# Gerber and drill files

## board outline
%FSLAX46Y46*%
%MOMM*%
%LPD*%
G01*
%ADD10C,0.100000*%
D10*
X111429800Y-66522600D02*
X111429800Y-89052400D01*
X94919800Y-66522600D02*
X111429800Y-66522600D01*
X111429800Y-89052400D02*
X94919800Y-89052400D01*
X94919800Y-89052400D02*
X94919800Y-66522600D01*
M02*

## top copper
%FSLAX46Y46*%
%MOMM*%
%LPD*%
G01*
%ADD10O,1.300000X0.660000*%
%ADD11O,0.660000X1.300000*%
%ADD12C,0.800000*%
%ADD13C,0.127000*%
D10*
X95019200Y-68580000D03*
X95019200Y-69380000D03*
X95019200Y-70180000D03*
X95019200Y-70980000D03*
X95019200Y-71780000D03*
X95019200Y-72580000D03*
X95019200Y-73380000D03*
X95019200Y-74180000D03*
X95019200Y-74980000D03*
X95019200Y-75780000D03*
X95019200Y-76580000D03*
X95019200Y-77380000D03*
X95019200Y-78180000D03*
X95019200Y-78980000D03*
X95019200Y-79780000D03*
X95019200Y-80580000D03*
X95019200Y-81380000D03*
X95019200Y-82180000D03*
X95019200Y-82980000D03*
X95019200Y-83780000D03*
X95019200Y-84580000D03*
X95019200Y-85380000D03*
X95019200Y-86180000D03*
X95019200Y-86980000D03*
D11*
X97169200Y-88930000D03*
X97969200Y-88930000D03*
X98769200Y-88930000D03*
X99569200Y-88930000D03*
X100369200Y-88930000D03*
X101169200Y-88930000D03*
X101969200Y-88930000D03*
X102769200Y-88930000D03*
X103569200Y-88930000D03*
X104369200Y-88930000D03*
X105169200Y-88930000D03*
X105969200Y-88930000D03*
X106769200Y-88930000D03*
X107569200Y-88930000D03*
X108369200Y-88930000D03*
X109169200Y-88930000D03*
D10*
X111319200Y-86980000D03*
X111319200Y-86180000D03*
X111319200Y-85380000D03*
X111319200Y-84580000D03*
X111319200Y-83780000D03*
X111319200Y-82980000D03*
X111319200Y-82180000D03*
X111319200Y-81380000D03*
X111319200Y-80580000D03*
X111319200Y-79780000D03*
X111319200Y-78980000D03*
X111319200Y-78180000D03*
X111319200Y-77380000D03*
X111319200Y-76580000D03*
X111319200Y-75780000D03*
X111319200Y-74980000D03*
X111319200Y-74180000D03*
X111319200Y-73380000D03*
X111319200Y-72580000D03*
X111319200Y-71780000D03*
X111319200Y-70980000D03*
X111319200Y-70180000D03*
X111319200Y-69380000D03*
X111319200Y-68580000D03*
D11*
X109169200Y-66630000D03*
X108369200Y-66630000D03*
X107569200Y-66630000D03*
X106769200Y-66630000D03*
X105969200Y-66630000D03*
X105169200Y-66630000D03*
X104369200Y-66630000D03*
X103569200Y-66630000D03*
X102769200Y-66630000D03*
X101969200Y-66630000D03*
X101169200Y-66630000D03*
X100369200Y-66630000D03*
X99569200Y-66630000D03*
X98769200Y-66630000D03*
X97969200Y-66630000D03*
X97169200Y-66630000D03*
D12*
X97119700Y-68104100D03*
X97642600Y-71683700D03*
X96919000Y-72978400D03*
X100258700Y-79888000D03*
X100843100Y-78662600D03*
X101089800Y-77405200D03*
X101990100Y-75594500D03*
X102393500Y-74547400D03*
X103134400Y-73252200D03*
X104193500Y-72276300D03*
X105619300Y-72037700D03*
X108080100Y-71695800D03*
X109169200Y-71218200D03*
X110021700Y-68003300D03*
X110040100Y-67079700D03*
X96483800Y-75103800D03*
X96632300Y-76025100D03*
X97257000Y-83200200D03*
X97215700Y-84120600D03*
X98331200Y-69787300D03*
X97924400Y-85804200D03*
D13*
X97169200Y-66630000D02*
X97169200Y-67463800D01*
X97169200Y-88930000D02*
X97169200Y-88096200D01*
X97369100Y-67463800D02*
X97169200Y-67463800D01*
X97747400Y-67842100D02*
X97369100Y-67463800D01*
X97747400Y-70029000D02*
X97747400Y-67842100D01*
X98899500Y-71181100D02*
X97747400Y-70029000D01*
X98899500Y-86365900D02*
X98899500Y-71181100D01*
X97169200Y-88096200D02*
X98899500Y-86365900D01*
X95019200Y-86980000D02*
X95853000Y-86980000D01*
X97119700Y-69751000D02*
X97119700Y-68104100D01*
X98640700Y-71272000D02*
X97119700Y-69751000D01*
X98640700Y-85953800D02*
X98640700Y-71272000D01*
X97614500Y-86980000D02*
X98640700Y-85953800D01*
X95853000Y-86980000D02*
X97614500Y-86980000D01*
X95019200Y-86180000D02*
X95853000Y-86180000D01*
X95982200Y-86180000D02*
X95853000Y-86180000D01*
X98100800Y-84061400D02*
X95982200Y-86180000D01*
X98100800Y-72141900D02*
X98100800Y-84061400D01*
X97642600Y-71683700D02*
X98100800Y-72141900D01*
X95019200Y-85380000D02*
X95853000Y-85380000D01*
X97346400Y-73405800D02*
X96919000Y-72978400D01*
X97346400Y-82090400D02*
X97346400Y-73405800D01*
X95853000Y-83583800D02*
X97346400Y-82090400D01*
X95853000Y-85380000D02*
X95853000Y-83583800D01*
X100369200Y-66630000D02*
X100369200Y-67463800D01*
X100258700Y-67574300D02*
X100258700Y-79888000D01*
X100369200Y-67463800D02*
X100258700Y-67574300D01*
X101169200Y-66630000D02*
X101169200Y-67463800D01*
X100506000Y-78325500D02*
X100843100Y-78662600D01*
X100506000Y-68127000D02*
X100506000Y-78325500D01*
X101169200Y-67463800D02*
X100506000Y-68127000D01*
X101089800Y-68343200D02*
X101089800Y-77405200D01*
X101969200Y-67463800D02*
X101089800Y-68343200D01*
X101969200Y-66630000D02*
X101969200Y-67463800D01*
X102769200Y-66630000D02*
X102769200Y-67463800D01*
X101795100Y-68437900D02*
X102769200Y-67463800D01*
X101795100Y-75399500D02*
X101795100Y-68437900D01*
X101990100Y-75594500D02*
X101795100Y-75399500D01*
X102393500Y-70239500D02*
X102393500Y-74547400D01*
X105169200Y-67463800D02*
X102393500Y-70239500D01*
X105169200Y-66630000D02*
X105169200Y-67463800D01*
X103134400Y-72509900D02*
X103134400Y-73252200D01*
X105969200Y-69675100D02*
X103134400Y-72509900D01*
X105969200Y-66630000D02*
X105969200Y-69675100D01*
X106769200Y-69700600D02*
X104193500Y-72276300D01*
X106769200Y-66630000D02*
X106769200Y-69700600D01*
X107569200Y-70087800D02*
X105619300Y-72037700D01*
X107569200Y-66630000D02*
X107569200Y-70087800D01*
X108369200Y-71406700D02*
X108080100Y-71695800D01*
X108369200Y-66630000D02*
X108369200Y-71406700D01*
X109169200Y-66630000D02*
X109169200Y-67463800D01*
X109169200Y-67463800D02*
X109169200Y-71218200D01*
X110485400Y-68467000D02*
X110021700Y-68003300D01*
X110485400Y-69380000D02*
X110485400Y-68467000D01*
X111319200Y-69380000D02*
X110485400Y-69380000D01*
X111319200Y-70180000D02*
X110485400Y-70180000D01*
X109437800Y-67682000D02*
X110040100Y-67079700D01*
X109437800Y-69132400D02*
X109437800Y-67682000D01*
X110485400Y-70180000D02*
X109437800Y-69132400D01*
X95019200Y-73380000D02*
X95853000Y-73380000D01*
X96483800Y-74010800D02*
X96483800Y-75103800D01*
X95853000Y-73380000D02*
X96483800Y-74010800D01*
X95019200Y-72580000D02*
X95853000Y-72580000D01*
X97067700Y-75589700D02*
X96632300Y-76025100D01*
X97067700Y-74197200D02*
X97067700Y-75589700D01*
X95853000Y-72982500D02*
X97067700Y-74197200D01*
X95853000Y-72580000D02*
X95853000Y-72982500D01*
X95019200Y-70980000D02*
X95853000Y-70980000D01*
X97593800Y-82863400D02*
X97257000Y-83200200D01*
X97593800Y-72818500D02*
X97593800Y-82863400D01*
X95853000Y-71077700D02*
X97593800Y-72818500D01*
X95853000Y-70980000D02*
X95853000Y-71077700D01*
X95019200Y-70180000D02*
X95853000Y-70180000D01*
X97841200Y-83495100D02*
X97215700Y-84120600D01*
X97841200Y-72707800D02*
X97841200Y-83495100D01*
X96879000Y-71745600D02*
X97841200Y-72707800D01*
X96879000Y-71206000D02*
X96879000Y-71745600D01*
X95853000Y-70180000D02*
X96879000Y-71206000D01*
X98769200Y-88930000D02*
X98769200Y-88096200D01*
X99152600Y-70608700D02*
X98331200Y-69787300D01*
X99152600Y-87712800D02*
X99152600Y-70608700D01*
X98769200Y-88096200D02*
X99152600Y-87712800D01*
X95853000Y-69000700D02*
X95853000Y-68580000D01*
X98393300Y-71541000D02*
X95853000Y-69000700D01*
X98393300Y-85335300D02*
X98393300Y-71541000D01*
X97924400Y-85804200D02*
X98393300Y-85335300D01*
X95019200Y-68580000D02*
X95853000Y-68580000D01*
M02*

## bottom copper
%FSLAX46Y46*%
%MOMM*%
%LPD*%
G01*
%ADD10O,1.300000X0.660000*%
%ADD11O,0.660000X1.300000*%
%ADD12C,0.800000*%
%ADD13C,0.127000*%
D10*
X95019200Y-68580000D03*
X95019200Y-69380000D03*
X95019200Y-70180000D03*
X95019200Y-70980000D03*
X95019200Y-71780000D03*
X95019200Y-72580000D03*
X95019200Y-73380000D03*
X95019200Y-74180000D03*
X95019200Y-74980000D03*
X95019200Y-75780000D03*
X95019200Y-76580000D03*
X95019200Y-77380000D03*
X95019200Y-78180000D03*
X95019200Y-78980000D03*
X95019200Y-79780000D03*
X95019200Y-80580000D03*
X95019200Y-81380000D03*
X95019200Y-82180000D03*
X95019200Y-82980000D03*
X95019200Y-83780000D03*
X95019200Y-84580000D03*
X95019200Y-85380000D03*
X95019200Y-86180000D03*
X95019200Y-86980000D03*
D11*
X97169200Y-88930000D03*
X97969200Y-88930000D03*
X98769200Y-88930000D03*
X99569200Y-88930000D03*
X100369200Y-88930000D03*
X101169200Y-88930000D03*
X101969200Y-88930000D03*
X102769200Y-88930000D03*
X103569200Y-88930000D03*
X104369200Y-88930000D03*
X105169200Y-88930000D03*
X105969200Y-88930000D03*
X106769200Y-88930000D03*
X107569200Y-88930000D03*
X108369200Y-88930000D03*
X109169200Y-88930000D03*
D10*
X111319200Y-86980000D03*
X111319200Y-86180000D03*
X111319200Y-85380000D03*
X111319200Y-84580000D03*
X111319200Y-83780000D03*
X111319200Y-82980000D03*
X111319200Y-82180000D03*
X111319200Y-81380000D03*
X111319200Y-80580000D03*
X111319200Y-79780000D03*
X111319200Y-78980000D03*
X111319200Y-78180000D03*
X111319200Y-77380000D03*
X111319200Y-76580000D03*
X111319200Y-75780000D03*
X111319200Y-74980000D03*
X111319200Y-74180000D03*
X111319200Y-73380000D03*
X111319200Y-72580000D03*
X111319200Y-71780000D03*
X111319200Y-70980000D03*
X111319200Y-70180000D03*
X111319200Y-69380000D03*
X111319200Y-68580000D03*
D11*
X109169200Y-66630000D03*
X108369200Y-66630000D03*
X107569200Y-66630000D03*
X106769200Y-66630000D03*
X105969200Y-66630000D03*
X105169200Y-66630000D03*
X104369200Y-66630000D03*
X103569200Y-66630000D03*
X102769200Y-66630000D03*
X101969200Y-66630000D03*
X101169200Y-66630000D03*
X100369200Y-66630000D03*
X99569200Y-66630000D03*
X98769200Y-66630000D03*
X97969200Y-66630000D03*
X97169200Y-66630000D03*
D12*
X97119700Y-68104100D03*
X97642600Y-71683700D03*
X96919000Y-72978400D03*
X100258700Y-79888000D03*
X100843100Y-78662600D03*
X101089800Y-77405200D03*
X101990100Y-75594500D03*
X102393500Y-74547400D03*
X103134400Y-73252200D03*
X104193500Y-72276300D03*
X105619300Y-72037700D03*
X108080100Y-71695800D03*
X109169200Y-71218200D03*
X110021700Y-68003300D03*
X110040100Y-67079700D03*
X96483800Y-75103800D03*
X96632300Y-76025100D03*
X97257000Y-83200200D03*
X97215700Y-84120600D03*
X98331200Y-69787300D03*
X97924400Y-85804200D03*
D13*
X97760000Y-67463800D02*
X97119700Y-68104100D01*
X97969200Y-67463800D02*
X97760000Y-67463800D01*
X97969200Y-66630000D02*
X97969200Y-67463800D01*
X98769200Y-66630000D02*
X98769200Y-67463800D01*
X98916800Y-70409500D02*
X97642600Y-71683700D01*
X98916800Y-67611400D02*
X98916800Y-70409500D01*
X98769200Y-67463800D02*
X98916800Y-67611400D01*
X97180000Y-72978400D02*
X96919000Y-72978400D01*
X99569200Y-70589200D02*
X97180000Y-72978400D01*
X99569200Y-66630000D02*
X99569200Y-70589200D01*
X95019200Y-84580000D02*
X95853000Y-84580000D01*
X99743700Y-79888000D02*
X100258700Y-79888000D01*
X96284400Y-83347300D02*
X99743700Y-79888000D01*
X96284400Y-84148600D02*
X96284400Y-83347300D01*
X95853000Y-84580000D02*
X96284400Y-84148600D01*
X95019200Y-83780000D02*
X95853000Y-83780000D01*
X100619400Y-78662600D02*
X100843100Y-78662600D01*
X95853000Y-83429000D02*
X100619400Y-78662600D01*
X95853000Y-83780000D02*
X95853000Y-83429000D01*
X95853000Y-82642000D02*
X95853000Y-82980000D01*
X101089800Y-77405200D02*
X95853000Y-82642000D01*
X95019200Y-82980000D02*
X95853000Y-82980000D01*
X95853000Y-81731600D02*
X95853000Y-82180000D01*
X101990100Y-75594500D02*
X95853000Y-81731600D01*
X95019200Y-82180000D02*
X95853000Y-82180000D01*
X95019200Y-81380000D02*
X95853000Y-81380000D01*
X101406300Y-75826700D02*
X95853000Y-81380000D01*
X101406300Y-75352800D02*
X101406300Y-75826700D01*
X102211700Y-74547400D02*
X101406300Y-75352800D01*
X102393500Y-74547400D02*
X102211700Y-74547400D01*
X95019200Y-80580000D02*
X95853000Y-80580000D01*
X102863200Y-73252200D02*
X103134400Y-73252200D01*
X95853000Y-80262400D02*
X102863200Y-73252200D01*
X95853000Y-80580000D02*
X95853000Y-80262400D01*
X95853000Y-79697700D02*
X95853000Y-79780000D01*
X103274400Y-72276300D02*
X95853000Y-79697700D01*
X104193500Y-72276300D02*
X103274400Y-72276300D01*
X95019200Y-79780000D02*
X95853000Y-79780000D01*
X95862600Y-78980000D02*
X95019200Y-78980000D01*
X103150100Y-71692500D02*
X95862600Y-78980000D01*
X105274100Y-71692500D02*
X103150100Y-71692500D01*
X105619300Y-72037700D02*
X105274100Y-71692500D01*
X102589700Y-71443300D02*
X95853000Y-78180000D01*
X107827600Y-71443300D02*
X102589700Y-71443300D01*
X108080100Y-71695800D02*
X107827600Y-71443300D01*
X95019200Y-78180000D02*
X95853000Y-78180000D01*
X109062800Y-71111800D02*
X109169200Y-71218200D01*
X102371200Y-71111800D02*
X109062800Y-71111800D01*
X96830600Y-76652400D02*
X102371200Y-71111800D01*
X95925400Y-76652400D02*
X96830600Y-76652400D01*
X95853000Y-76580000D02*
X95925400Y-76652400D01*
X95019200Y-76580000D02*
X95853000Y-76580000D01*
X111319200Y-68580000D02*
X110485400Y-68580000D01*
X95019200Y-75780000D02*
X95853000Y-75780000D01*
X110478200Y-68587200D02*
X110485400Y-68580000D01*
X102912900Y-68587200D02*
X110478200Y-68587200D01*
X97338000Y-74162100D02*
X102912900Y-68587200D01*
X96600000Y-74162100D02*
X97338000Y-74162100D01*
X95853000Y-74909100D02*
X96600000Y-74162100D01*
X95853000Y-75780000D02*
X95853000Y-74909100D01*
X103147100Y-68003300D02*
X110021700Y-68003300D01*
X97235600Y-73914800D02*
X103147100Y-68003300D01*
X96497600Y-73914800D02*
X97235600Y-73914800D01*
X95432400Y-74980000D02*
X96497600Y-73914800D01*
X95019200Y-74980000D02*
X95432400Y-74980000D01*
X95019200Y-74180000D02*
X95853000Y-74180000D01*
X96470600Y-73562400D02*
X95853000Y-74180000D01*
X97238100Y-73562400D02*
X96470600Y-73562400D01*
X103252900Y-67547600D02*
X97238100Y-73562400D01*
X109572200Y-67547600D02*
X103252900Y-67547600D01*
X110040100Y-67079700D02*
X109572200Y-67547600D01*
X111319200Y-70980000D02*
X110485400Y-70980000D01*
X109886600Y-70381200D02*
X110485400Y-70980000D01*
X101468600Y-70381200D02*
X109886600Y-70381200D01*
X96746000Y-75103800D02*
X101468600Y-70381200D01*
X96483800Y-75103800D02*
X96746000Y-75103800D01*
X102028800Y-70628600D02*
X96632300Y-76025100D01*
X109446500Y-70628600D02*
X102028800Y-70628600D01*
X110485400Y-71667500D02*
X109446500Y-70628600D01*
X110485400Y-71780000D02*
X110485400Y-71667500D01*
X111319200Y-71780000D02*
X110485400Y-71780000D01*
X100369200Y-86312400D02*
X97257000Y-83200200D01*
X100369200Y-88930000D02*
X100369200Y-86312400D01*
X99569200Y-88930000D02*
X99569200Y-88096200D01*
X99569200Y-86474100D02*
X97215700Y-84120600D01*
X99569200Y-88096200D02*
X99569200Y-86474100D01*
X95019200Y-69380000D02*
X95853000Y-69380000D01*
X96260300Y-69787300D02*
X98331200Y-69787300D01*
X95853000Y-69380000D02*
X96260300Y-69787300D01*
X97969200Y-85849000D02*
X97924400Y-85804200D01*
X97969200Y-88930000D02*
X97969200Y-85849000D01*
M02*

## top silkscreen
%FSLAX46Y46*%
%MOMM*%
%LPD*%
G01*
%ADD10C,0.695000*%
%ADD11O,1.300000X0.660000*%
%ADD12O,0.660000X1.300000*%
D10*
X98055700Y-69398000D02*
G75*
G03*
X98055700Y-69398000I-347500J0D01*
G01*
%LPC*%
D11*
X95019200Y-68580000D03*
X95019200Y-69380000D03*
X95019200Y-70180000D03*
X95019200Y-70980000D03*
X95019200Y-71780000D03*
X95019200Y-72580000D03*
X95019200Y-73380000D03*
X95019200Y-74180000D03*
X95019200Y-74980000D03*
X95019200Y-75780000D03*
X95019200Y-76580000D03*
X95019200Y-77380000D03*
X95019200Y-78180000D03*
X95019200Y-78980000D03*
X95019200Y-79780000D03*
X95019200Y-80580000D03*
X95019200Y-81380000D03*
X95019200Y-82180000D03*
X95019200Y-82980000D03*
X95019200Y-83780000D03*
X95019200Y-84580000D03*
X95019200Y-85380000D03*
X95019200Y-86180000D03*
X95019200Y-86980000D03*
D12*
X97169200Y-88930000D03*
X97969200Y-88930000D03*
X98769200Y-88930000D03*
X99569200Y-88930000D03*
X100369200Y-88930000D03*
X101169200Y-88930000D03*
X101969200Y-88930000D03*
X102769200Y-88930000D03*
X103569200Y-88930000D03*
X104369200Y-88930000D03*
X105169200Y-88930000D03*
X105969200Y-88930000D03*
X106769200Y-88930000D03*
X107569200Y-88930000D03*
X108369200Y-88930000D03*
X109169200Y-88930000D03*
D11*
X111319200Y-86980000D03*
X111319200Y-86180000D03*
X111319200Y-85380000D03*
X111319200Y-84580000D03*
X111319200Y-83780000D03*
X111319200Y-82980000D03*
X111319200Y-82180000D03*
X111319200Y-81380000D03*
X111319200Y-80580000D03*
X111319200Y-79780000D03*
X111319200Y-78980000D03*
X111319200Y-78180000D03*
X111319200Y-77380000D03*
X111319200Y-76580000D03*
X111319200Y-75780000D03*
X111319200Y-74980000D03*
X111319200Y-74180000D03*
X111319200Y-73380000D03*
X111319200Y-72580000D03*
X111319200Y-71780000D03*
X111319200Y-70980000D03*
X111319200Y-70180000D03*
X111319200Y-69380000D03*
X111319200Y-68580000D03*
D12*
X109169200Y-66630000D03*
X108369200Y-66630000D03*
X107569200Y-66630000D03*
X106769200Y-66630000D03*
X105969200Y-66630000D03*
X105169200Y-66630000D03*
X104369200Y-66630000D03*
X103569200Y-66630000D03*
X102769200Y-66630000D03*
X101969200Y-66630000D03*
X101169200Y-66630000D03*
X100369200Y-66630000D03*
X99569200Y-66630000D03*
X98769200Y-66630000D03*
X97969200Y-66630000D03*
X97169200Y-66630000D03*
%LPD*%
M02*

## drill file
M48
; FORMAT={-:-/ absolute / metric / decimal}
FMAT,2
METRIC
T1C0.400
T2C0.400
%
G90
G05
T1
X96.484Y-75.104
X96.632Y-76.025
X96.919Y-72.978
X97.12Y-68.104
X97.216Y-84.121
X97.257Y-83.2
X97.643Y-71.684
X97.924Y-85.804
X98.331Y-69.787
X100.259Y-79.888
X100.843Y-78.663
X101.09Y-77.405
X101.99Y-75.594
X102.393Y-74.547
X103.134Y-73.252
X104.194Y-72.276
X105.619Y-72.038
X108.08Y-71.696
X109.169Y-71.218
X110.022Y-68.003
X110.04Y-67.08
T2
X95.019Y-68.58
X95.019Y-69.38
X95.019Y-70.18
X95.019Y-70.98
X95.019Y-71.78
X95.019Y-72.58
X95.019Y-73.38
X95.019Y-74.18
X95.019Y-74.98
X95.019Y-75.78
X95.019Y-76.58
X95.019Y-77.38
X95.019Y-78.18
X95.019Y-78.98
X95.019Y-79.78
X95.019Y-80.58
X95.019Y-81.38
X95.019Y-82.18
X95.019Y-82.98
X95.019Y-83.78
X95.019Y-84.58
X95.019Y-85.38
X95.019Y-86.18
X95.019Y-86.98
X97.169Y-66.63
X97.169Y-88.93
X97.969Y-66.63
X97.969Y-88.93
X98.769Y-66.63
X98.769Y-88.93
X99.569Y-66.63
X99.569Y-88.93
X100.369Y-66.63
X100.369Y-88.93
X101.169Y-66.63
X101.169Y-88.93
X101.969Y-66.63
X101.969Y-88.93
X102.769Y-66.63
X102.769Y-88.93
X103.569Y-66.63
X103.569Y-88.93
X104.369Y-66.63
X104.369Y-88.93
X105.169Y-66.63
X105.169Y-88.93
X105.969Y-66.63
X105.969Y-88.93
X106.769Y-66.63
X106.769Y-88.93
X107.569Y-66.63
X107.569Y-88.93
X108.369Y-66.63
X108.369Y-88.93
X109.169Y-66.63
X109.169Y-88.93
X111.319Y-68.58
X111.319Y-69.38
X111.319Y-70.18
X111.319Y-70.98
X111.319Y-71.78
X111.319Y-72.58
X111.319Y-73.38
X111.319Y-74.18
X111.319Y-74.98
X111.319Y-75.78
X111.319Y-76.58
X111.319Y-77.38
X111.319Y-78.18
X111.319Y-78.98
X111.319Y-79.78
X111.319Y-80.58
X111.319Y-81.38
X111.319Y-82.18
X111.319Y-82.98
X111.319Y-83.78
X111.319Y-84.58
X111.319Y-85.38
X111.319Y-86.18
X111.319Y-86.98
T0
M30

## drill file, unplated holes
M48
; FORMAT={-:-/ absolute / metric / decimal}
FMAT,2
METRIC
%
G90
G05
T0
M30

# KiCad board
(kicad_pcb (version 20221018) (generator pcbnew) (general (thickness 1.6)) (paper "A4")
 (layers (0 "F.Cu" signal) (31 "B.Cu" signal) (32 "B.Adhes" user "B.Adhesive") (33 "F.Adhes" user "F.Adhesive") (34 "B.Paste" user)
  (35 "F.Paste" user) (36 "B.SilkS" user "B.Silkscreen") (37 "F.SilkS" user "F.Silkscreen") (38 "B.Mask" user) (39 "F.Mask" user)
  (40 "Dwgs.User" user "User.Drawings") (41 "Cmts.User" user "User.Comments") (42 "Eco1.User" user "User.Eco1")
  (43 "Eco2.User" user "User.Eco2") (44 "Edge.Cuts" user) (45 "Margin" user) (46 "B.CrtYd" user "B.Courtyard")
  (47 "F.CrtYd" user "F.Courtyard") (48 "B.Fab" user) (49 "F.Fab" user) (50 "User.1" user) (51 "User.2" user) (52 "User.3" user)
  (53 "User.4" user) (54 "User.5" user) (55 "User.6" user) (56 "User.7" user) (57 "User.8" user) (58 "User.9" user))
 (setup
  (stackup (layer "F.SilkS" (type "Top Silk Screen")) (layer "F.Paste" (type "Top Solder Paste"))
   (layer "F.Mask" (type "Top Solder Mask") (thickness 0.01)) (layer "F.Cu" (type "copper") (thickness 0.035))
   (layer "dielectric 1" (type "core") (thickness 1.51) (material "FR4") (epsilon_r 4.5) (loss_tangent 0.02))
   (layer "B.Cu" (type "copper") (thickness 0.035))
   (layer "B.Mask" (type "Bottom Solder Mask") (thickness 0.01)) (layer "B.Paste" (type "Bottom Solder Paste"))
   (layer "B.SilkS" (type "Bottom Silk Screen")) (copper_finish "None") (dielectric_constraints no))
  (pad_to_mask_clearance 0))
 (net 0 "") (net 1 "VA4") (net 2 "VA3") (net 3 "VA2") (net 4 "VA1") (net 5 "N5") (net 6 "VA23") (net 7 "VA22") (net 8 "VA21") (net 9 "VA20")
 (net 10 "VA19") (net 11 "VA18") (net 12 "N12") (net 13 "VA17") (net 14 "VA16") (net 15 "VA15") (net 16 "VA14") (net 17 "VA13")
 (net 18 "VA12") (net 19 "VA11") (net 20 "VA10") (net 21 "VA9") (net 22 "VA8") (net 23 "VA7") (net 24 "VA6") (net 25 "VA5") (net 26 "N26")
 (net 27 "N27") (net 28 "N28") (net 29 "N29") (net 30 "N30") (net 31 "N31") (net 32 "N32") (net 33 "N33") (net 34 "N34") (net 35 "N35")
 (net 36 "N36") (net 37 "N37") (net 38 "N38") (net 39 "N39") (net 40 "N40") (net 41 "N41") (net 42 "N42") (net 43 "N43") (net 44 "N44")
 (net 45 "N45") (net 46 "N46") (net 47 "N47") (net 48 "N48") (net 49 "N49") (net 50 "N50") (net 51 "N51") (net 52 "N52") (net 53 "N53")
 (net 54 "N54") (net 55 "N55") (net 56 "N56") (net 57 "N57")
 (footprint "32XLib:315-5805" (layer "F.Cu") (at 103.1692 77.78)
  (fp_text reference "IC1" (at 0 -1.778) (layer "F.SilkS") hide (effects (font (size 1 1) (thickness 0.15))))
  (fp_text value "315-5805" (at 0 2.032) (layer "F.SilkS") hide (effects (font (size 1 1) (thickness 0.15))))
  (fp_circle (center -5.461 -8.382) (end -4.826 -8.382) (stroke (width 0.12) (type solid)) (fill solid) (layer "F.SilkS"))
  (pad "1" thru_hole oval (at -8.15 -9.2) (size 1.3 0.66) (drill 0.4) (layers "*.Cu" "*.Mask") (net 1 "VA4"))
  (pad "2" thru_hole oval (at -8.15 -8.4) (size 1.3 0.66) (drill 0.4) (layers "*.Cu" "*.Mask") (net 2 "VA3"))
  (pad "3" thru_hole oval (at -8.15 -7.6) (size 1.3 0.66) (drill 0.4) (layers "*.Cu" "*.Mask") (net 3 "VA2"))
  (pad "4" thru_hole oval (at -8.15 -6.8) (size 1.3 0.66) (drill 0.4) (layers "*.Cu" "*.Mask") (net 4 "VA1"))
  (pad "5" thru_hole oval (at -8.15 -6) (size 1.3 0.66) (drill 0.4) (layers "*.Cu" "*.Mask") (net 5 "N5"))
  (pad "6" thru_hole oval (at -8.15 -5.2) (size 1.3 0.66) (drill 0.4) (layers "*.Cu" "*.Mask") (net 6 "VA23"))
  (pad "7" thru_hole oval (at -8.15 -4.4) (size 1.3 0.66) (drill 0.4) (layers "*.Cu" "*.Mask") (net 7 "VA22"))
  (pad "8" thru_hole oval (at -8.15 -3.6) (size 1.3 0.66) (drill 0.4) (layers "*.Cu" "*.Mask") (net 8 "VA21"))
  (pad "9" thru_hole oval (at -8.15 -2.8) (size 1.3 0.66) (drill 0.4) (layers "*.Cu" "*.Mask") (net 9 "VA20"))
  (pad "10" thru_hole oval (at -8.15 -2) (size 1.3 0.66) (drill 0.4) (layers "*.Cu" "*.Mask") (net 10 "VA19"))
  (pad "11" thru_hole oval (at -8.15 -1.2) (size 1.3 0.66) (drill 0.4) (layers "*.Cu" "*.Mask") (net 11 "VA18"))
  (pad "12" thru_hole oval (at -8.15 -0.4) (size 1.3 0.66) (drill 0.4) (layers "*.Cu" "*.Mask") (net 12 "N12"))
  (pad "13" thru_hole oval (at -8.15 0.4) (size 1.3 0.66) (drill 0.4) (layers "*.Cu" "*.Mask") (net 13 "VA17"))
  (pad "14" thru_hole oval (at -8.15 1.2) (size 1.3 0.66) (drill 0.4) (layers "*.Cu" "*.Mask") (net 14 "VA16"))
  (pad "15" thru_hole oval (at -8.15 2) (size 1.3 0.66) (drill 0.4) (layers "*.Cu" "*.Mask") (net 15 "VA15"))
  (pad "16" thru_hole oval (at -8.15 2.8) (size 1.3 0.66) (drill 0.4) (layers "*.Cu" "*.Mask") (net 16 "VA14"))
  (pad "17" thru_hole oval (at -8.15 3.6) (size 1.3 0.66) (drill 0.4) (layers "*.Cu" "*.Mask") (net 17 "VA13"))
  (pad "18" thru_hole oval (at -8.15 4.4) (size 1.3 0.66) (drill 0.4) (layers "*.Cu" "*.Mask") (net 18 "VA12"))
  (pad "19" thru_hole oval (at -8.15 5.2) (size 1.3 0.66) (drill 0.4) (layers "*.Cu" "*.Mask") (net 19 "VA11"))
  (pad "20" thru_hole oval (at -8.15 6) (size 1.3 0.66) (drill 0.4) (layers "*.Cu" "*.Mask") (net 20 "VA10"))
  (pad "21" thru_hole oval (at -8.15 6.8) (size 1.3 0.66) (drill 0.4) (layers "*.Cu" "*.Mask") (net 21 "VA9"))
  (pad "22" thru_hole oval (at -8.15 7.6) (size 1.3 0.66) (drill 0.4) (layers "*.Cu" "*.Mask") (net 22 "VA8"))
  (pad "23" thru_hole oval (at -8.15 8.4) (size 1.3 0.66) (drill 0.4) (layers "*.Cu" "*.Mask") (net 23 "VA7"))
  (pad "24" thru_hole oval (at -8.15 9.2) (size 1.3 0.66) (drill 0.4) (layers "*.Cu" "*.Mask") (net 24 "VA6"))
  (pad "25" thru_hole oval (at -6 11.15 90) (size 1.3 0.66) (drill 0.4) (layers "*.Cu" "*.Mask") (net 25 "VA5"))
  (pad "26" thru_hole oval (at -5.2 11.15 90) (size 1.3 0.66) (drill 0.4) (layers "*.Cu" "*.Mask") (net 1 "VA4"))
  (pad "27" thru_hole oval (at -4.4 11.15 90) (size 1.3 0.66) (drill 0.4) (layers "*.Cu" "*.Mask") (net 2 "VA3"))
  (pad "28" thru_hole oval (at -3.6 11.15 90) (size 1.3 0.66) (drill 0.4) (layers "*.Cu" "*.Mask") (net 3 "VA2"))
  (pad "29" thru_hole oval (at -2.8 11.15 90) (size 1.3 0.66) (drill 0.4) (layers "*.Cu" "*.Mask") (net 4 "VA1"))
  (pad "30" thru_hole oval (at -2 11.15 90) (size 1.3 0.66) (drill 0.4) (layers "*.Cu" "*.Mask") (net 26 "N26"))
  (pad "31" thru_hole oval (at -1.2 11.15 90) (size 1.3 0.66) (drill 0.4) (layers "*.Cu" "*.Mask") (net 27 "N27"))
  (pad "32" thru_hole oval (at -0.4 11.15 90) (size 1.3 0.66) (drill 0.4) (layers "*.Cu" "*.Mask") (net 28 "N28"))
  (pad "33" thru_hole oval (at 0.4 11.15 90) (size 1.3 0.66) (drill 0.4) (layers "*.Cu" "*.Mask") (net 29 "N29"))
  (pad "34" thru_hole oval (at 1.2 11.15 90) (size 1.3 0.66) (drill 0.4) (layers "*.Cu" "*.Mask") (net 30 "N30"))
  (pad "35" thru_hole oval (at 2 11.15 90) (size 1.3 0.66) (drill 0.4) (layers "*.Cu" "*.Mask") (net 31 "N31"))
  (pad "36" thru_hole oval (at 2.8 11.15 90) (size 1.3 0.66) (drill 0.4) (layers "*.Cu" "*.Mask") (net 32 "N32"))
  (pad "37" thru_hole oval (at 3.6 11.15 90) (size 1.3 0.66) (drill 0.4) (layers "*.Cu" "*.Mask") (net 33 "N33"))
  (pad "38" thru_hole oval (at 4.4 11.15 90) (size 1.3 0.66) (drill 0.4) (layers "*.Cu" "*.Mask") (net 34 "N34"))
  (pad "39" thru_hole oval (at 5.2 11.15 90) (size 1.3 0.66) (drill 0.4) (layers "*.Cu" "*.Mask") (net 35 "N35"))
  (pad "40" thru_hole oval (at 6 11.15 90) (size 1.3 0.66) (drill 0.4) (layers "*.Cu" "*.Mask") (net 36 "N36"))
  (pad "41" thru_hole oval (at 8.15 9.2) (size 1.3 0.66) (drill 0.4) (layers "*.Cu" "*.Mask") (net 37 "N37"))
  (pad "42" thru_hole oval (at 8.15 8.4) (size 1.3 0.66) (drill 0.4) (layers "*.Cu" "*.Mask") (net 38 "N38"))
  (pad "43" thru_hole oval (at 8.15 7.6) (size 1.3 0.66) (drill 0.4) (layers "*.Cu" "*.Mask") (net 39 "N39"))
  (pad "44" thru_hole oval (at 8.15 6.8) (size 1.3 0.66) (drill 0.4) (layers "*.Cu" "*.Mask") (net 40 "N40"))
  (pad "45" thru_hole oval (at 8.15 6) (size 1.3 0.66) (drill 0.4) (layers "*.Cu" "*.Mask") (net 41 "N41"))
  (pad "46" thru_hole oval (at 8.15 5.2) (size 1.3 0.66) (drill 0.4) (layers "*.Cu" "*.Mask") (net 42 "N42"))
  (pad "47" thru_hole oval (at 8.15 4.4) (size 1.3 0.66) (drill 0.4) (layers "*.Cu" "*.Mask") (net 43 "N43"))
  (pad "48" thru_hole oval (at 8.15 3.6) (size 1.3 0.66) (drill 0.4) (layers "*.Cu" "*.Mask") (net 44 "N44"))
  (pad "49" thru_hole oval (at 8.15 2.8) (size 1.3 0.66) (drill 0.4) (layers "*.Cu" "*.Mask") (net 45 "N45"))
  (pad "50" thru_hole oval (at 8.15 2) (size 1.3 0.66) (drill 0.4) (layers "*.Cu" "*.Mask") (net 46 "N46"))
  (pad "51" thru_hole oval (at 8.15 1.2) (size 1.3 0.66) (drill 0.4) (layers "*.Cu" "*.Mask") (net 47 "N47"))
  (pad "52" thru_hole oval (at 8.15 0.4) (size 1.3 0.66) (drill 0.4) (layers "*.Cu" "*.Mask") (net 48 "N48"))
  (pad "53" thru_hole oval (at 8.15 -0.4) (size 1.3 0.66) (drill 0.4) (layers "*.Cu" "*.Mask") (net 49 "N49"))
  (pad "54" thru_hole oval (at 8.15 -1.2) (size 1.3 0.66) (drill 0.4) (layers "*.Cu" "*.Mask") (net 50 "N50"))
  (pad "55" thru_hole oval (at 8.15 -2) (size 1.3 0.66) (drill 0.4) (layers "*.Cu" "*.Mask") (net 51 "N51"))
  (pad "56" thru_hole oval (at 8.15 -2.8) (size 1.3 0.66) (drill 0.4) (layers "*.Cu" "*.Mask") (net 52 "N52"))
  (pad "57" thru_hole oval (at 8.15 -3.6) (size 1.3 0.66) (drill 0.4) (layers "*.Cu" "*.Mask") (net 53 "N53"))
  (pad "58" thru_hole oval (at 8.15 -4.4) (size 1.3 0.66) (drill 0.4) (layers "*.Cu" "*.Mask") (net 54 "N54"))
  (pad "59" thru_hole oval (at 8.15 -5.2) (size 1.3 0.66) (drill 0.4) (layers "*.Cu" "*.Mask") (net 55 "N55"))
  (pad "60" thru_hole oval (at 8.15 -6) (size 1.3 0.66) (drill 0.4) (layers "*.Cu" "*.Mask") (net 6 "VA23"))
  (pad "61" thru_hole oval (at 8.15 -6.8) (size 1.3 0.66) (drill 0.4) (layers "*.Cu" "*.Mask") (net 7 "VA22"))
  (pad "62" thru_hole oval (at 8.15 -7.6) (size 1.3 0.66) (drill 0.4) (layers "*.Cu" "*.Mask") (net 8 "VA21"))
  (pad "63" thru_hole oval (at 8.15 -8.4) (size 1.3 0.66) (drill 0.4) (layers "*.Cu" "*.Mask") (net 9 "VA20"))
  (pad "64" thru_hole oval (at 8.15 -9.2) (size 1.3 0.66) (drill 0.4) (layers "*.Cu" "*.Mask") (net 10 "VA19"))
  (pad "65" thru_hole oval (at 6 -11.15 90) (size 1.3 0.66) (drill 0.4) (layers "*.Cu" "*.Mask") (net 11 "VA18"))
  (pad "66" thru_hole oval (at 5.2 -11.15 90) (size 1.3 0.66) (drill 0.4) (layers "*.Cu" "*.Mask") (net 13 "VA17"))
  (pad "67" thru_hole oval (at 4.4 -11.15 90) (size 1.3 0.66) (drill 0.4) (layers "*.Cu" "*.Mask") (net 14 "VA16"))
  (pad "68" thru_hole oval (at 3.6 -11.15 90) (size 1.3 0.66) (drill 0.4) (layers "*.Cu" "*.Mask") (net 15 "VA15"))
  (pad "69" thru_hole oval (at 2.8 -11.15 90) (size 1.3 0.66) (drill 0.4) (layers "*.Cu" "*.Mask") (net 16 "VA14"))
  (pad "70" thru_hole oval (at 2 -11.15 90) (size 1.3 0.66) (drill 0.4) (layers "*.Cu" "*.Mask") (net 17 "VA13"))
  (pad "71" thru_hole oval (at 1.2 -11.15 90) (size 1.3 0.66) (drill 0.4) (layers "*.Cu" "*.Mask") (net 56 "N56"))
  (pad "72" thru_hole oval (at 0.4 -11.15 90) (size 1.3 0.66) (drill 0.4) (layers "*.Cu" "*.Mask") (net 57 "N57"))
  (pad "73" thru_hole oval (at -0.4 -11.15 90) (size 1.3 0.66) (drill 0.4) (layers "*.Cu" "*.Mask") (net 18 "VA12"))
  (pad "74" thru_hole oval (at -1.2 -11.15 90) (size 1.3 0.66) (drill 0.4) (layers "*.Cu" "*.Mask") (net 19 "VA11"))
  (pad "75" thru_hole oval (at -2 -11.15 90) (size 1.3 0.66) (drill 0.4) (layers "*.Cu" "*.Mask") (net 20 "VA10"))
  (pad "76" thru_hole oval (at -2.8 -11.15 90) (size 1.3 0.66) (drill 0.4) (layers "*.Cu" "*.Mask") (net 21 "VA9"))
  (pad "77" thru_hole oval (at -3.6 -11.15 90) (size 1.3 0.66) (drill 0.4) (layers "*.Cu" "*.Mask") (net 22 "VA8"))
  (pad "78" thru_hole oval (at -4.4 -11.15 90) (size 1.3 0.66) (drill 0.4) (layers "*.Cu" "*.Mask") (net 23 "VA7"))
  (pad "79" thru_hole oval (at -5.2 -11.15 90) (size 1.3 0.66) (drill 0.4) (layers "*.Cu" "*.Mask") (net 24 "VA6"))
  (pad "80" thru_hole oval (at -6 -11.15 90) (size 1.3 0.66) (drill 0.4) (layers "*.Cu" "*.Mask") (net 25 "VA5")))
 (gr_line (start 94.9198 89.0524) (end 94.9198 66.5226) (stroke (width 0.1) (type default)) (layer "Edge.Cuts"))
 (gr_line (start 111.4298 66.5226) (end 111.4298 89.0524) (stroke (width 0.1) (type default)) (layer "Edge.Cuts"))
 (gr_line (start 94.9198 66.5226) (end 111.4298 66.5226) (stroke (width 0.1) (type default)) (layer "Edge.Cuts"))
 (gr_line (start 111.4298 89.0524) (end 94.9198 89.0524) (stroke (width 0.1) (type default)) (layer "Edge.Cuts"))
 (segment (start 98.3933 71.541) (end 95.853 69.0007) (width 0.127) (layer "F.Cu") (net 1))
 (segment (start 98.3933 85.3353) (end 98.3933 71.541) (width 0.127) (layer "F.Cu") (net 1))
 (segment (start 95.853 69.0007) (end 95.853 68.58) (width 0.127) (layer "F.Cu") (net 1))
 (segment (start 95.0192 68.58) (end 95.853 68.58) (width 0.127) (layer "F.Cu") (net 1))
 (segment (start 97.9244 85.8042) (end 98.3933 85.3353) (width 0.127) (layer "F.Cu") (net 1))
 (via (at 97.9244 85.8042) (size 0.8) (drill 0.4) (layers "F.Cu" "B.Cu") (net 1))
 (segment (start 97.9692 85.849) (end 97.9244 85.8042) (width 0.127) (layer "B.Cu") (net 1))
 (segment (start 97.9692 88.93) (end 97.9692 85.849) (width 0.127) (layer "B.Cu") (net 1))
 (segment (start 98.7692 88.93) (end 98.7692 88.0962) (width 0.127) (layer "F.Cu") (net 2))
 (segment (start 98.7692 88.0962) (end 99.1526 87.7128) (width 0.127) (layer "F.Cu") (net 2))
 (segment (start 99.1526 70.6087) (end 98.3312 69.7873) (width 0.127) (layer "F.Cu") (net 2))
 (segment (start 99.1526 87.7128) (end 99.1526 70.6087) (width 0.127) (layer "F.Cu") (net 2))
 (via (at 98.3312 69.7873) (size 0.8) (drill 0.4) (layers "F.Cu" "B.Cu") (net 2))
 (segment (start 95.853 69.38) (end 96.2603 69.7873) (width 0.127) (layer "B.Cu") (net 2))
 (segment (start 95.0192 69.38) (end 95.853 69.38) (width 0.127) (layer "B.Cu") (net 2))
 (segment (start 96.2603 69.7873) (end 98.3312 69.7873) (width 0.127) (layer "B.Cu") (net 2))
 (segment (start 95.853 70.18) (end 96.879 71.206) (width 0.127) (layer "F.Cu") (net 3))
 (segment (start 97.8412 72.7078) (end 97.8412 83.4951) (width 0.127) (layer "F.Cu") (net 3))
 (segment (start 96.879 71.206) (end 96.879 71.7456) (width 0.127) (layer "F.Cu") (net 3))
 (segment (start 95.0192 70.18) (end 95.853 70.18) (width 0.127) (layer "F.Cu") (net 3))
 (segment (start 96.879 71.7456) (end 97.8412 72.7078) (width 0.127) (layer "F.Cu") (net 3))
 (segment (start 97.8412 83.4951) (end 97.2157 84.1206) (width 0.127) (layer "F.Cu") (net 3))
 (via (at 97.2157 84.1206) (size 0.8) (drill 0.4) (layers "F.Cu" "B.Cu") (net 3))
 (segment (start 99.5692 88.0962) (end 99.5692 86.4741) (width 0.127) (layer "B.Cu") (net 3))
 (segment (start 99.5692 86.4741) (end 97.2157 84.1206) (width 0.127) (layer "B.Cu") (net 3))
 (segment (start 99.5692 88.93) (end 99.5692 88.0962) (width 0.127) (layer "B.Cu") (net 3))
 (segment (start 97.5938 82.8634) (end 97.257 83.2002) (width 0.127) (layer "F.Cu") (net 4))
 (segment (start 97.5938 72.8185) (end 97.5938 82.8634) (width 0.127) (layer "F.Cu") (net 4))
 (segment (start 95.853 71.0777) (end 97.5938 72.8185) (width 0.127) (layer "F.Cu") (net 4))
 (segment (start 95.0192 70.98) (end 95.853 70.98) (width 0.127) (layer "F.Cu") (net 4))
 (segment (start 95.853 70.98) (end 95.853 71.0777) (width 0.127) (layer "F.Cu") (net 4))
 (via (at 97.257 83.2002) (size 0.8) (drill 0.4) (layers "F.Cu" "B.Cu") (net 4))
 (segment (start 100.3692 86.3124) (end 97.257 83.2002) (width 0.127) (layer "B.Cu") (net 4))
 (segment (start 100.3692 88.93) (end 100.3692 86.3124) (width 0.127) (layer "B.Cu") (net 4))
 (segment (start 95.853 72.58) (end 95.853 72.9825) (width 0.127) (layer "F.Cu") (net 6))
 (segment (start 95.853 72.9825) (end 97.0677 74.1972) (width 0.127) (layer "F.Cu") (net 6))
 (segment (start 95.0192 72.58) (end 95.853 72.58) (width 0.127) (layer "F.Cu") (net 6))
 (segment (start 97.0677 74.1972) (end 97.0677 75.5897) (width 0.127) (layer "F.Cu") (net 6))
 (segment (start 97.0677 75.5897) (end 96.6323 76.0251) (width 0.127) (layer "F.Cu") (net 6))
 (via (at 96.6323 76.0251) (size 0.8) (drill 0.4) (layers "F.Cu" "B.Cu") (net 6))
 (segment (start 111.3192 71.78) (end 110.4854 71.78) (width 0.127) (layer "B.Cu") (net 6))
 (segment (start 110.4854 71.78) (end 110.4854 71.6675) (width 0.127) (layer "B.Cu") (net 6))
 (segment (start 109.4465 70.6286) (end 102.0288 70.6286) (width 0.127) (layer "B.Cu") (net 6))
 (segment (start 102.0288 70.6286) (end 96.6323 76.0251) (width 0.127) (layer "B.Cu") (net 6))
 (segment (start 110.4854 71.6675) (end 109.4465 70.6286) (width 0.127) (layer "B.Cu") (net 6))
 (segment (start 95.0192 73.38) (end 95.853 73.38) (width 0.127) (layer "F.Cu") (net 7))
 (segment (start 96.4838 74.0108) (end 96.4838 75.1038) (width 0.127) (layer "F.Cu") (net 7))
 (segment (start 95.853 73.38) (end 96.4838 74.0108) (width 0.127) (layer "F.Cu") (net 7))
 (via (at 96.4838 75.1038) (size 0.8) (drill 0.4) (layers "F.Cu" "B.Cu") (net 7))
 (segment (start 96.746 75.1038) (end 101.4686 70.3812) (width 0.127) (layer "B.Cu") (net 7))
 (segment (start 96.4838 75.1038) (end 96.746 75.1038) (width 0.127) (layer "B.Cu") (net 7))
 (segment (start 111.3192 70.98) (end 110.4854 70.98) (width 0.127) (layer "B.Cu") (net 7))
 (segment (start 101.4686 70.3812) (end 109.8866 70.3812) (width 0.127) (layer "B.Cu") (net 7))
 (segment (start 109.8866 70.3812) (end 110.4854 70.98) (width 0.127) (layer "B.Cu") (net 7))
 (segment (start 109.4378 69.1324) (end 109.4378 67.682) (width 0.127) (layer "F.Cu") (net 8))
 (segment (start 109.4378 67.682) (end 110.0401 67.0797) (width 0.127) (layer "F.Cu") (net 8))
 (segment (start 110.4854 70.18) (end 109.4378 69.1324) (width 0.127) (layer "F.Cu") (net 8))
 (segment (start 111.3192 70.18) (end 110.4854 70.18) (width 0.127) (layer "F.Cu") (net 8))
 (via (at 110.0401 67.0797) (size 0.8) (drill 0.4) (layers "F.Cu" "B.Cu") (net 8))
 (segment (start 96.4706 73.5624) (end 95.853 74.18) (width 0.127) (layer "B.Cu") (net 8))
 (segment (start 95.0192 74.18) (end 95.853 74.18) (width 0.127) (layer "B.Cu") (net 8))
 (segment (start 103.2529 67.5476) (end 97.2381 73.5624) (width 0.127) (layer "B.Cu") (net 8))
 (segment (start 109.5722 67.5476) (end 103.2529 67.5476) (width 0.127) (layer "B.Cu") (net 8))
 (segment (start 110.0401 67.0797) (end 109.5722 67.5476) (width 0.127) (layer "B.Cu") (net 8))
 (segment (start 97.2381 73.5624) (end 96.4706 73.5624) (width 0.127) (layer "B.Cu") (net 8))
 (segment (start 110.4854 68.467) (end 110.0217 68.0033) (width 0.127) (layer "F.Cu") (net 9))
 (segment (start 110.4854 69.38) (end 110.4854 68.467) (width 0.127) (layer "F.Cu") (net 9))
 (segment (start 111.3192 69.38) (end 110.4854 69.38) (width 0.127) (layer "F.Cu") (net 9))
 (via (at 110.0217 68.0033) (size 0.8) (drill 0.4) (layers "F.Cu" "B.Cu") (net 9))
 (segment (start 103.1471 68.0033) (end 110.0217 68.0033) (width 0.127) (layer "B.Cu") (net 9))
 (segment (start 97.2356 73.9148) (end 103.1471 68.0033) (width 0.127) (layer "B.Cu") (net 9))
 (segment (start 96.4976 73.9148) (end 97.2356 73.9148) (width 0.127) (layer "B.Cu") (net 9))
 (segment (start 95.4324 74.98) (end 96.4976 73.9148) (width 0.127) (layer "B.Cu") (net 9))
 (segment (start 95.0192 74.98) (end 95.4324 74.98) (width 0.127) (layer "B.Cu") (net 9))
 (segment (start 97.338 74.1621) (end 102.9129 68.5872) (width 0.127) (layer "B.Cu") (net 10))
 (segment (start 110.4782 68.5872) (end 110.4854 68.58) (width 0.127) (layer "B.Cu") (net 10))
 (segment (start 102.9129 68.5872) (end 110.4782 68.5872) (width 0.127) (layer "B.Cu") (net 10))
 (segment (start 95.853 75.78) (end 95.853 74.9091) (width 0.127) (layer "B.Cu") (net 10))
 (segment (start 111.3192 68.58) (end 110.4854 68.58) (width 0.127) (layer "B.Cu") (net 10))
 (segment (start 95.853 74.9091) (end 96.6 74.1621) (width 0.127) (layer "B.Cu") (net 10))
 (segment (start 96.6 74.1621) (end 97.338 74.1621) (width 0.127) (layer "B.Cu") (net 10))
 (segment (start 95.0192 75.78) (end 95.853 75.78) (width 0.127) (layer "B.Cu") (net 10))
 (segment (start 109.1692 67.4638) (end 109.1692 71.2182) (width 0.127) (layer "F.Cu") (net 11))
 (segment (start 109.1692 66.63) (end 109.1692 67.4638) (width 0.127) (layer "F.Cu") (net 11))
 (via (at 109.1692 71.2182) (size 0.8) (drill 0.4) (layers "F.Cu" "B.Cu") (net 11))
 (segment (start 95.0192 76.58) (end 95.853 76.58) (width 0.127) (layer "B.Cu") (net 11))
 (segment (start 95.853 76.58) (end 95.9254 76.6524) (width 0.127) (layer "B.Cu") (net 11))
 (segment (start 95.9254 76.6524) (end 96.8306 76.6524) (width 0.127) (layer "B.Cu") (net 11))
 (segment (start 109.0628 71.1118) (end 109.1692 71.2182) (width 0.127) (layer "B.Cu") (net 11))
 (segment (start 96.8306 76.6524) (end 102.3712 71.1118) (width 0.127) (layer "B.Cu") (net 11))
 (segment (start 102.3712 71.1118) (end 109.0628 71.1118) (width 0.127) (layer "B.Cu") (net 11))
 (segment (start 108.3692 66.63) (end 108.3692 71.4067) (width 0.127) (layer "F.Cu") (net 13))
 (segment (start 108.3692 71.4067) (end 108.0801 71.6958) (width 0.127) (layer "F.Cu") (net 13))
 (via (at 108.0801 71.6958) (size 0.8) (drill 0.4) (layers "F.Cu" "B.Cu") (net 13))
 (segment (start 102.5897 71.4433) (end 95.853 78.18) (width 0.127) (layer "B.Cu") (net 13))
 (segment (start 107.8276 71.4433) (end 102.5897 71.4433) (width 0.127) (layer "B.Cu") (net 13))
 (segment (start 108.0801 71.6958) (end 107.8276 71.4433) (width 0.127) (layer "B.Cu") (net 13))
 (segment (start 95.0192 78.18) (end 95.853 78.18) (width 0.127) (layer "B.Cu") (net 13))
 (segment (start 107.5692 66.63) (end 107.5692 70.0878) (width 0.127) (layer "F.Cu") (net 14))
 (segment (start 107.5692 70.0878) (end 105.6193 72.0377) (width 0.127) (layer "F.Cu") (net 14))
 (via (at 105.6193 72.0377) (size 0.8) (drill 0.4) (layers "F.Cu" "B.Cu") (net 14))
 (segment (start 105.6193 72.0377) (end 105.2741 71.6925) (width 0.127) (layer "B.Cu") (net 14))
 (segment (start 105.2741 71.6925) (end 103.1501 71.6925) (width 0.127) (layer "B.Cu") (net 14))
 (segment (start 95.8626 78.98) (end 95.0192 78.98) (width 0.127) (layer "B.Cu") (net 14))
 (segment (start 103.1501 71.6925) (end 95.8626 78.98) (width 0.127) (layer "B.Cu") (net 14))
 (segment (start 106.7692 69.7006) (end 104.1935 72.2763) (width 0.127) (layer "F.Cu") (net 15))
 (segment (start 106.7692 66.63) (end 106.7692 69.7006) (width 0.127) (layer "F.Cu") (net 15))
 (via (at 104.1935 72.2763) (size 0.8) (drill 0.4) (layers "F.Cu" "B.Cu") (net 15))
 (segment (start 104.1935 72.2763) (end 103.2744 72.2763) (width 0.127) (layer "B.Cu") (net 15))
 (segment (start 95.0192 79.78) (end 95.853 79.78) (width 0.127) (layer "B.Cu") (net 15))
 (segment (start 103.2744 72.2763) (end 95.853 79.6977) (width 0.127) (layer "B.Cu") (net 15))
 (segment (start 95.853 79.6977) (end 95.853 79.78) (width 0.127) (layer "B.Cu") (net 15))
 (segment (start 105.9692 66.63) (end 105.9692 69.6751) (width 0.127) (layer "F.Cu") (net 16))
 (segment (start 105.9692 69.6751) (end 103.1344 72.5099) (width 0.127) (layer "F.Cu") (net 16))
 (segment (start 103.1344 72.5099) (end 103.1344 73.2522) (width 0.127) (layer "F.Cu") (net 16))
 (via (at 103.1344 73.2522) (size 0.8) (drill 0.4) (layers "F.Cu" "B.Cu") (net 16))
 (segment (start 95.0192 80.58) (end 95.853 80.58) (width 0.127) (layer "B.Cu") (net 16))
 (segment (start 95.853 80.58) (end 95.853 80.2624) (width 0.127) (layer "B.Cu") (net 16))
 (segment (start 95.853 80.2624) (end 102.8632 73.2522) (width 0.127) (layer "B.Cu") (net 16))
 (segment (start 102.8632 73.2522) (end 103.1344 73.2522) (width 0.127) (layer "B.Cu") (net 16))
 (segment (start 105.1692 67.4638) (end 102.3935 70.2395) (width 0.127) (layer "F.Cu") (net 17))
 (segment (start 105.1692 66.63) (end 105.1692 67.4638) (width 0.127) (layer "F.Cu") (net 17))
 (segment (start 102.3935 70.2395) (end 102.3935 74.5474) (width 0.127) (layer "F.Cu") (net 17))
 (via (at 102.3935 74.5474) (size 0.8) (drill 0.4) (layers "F.Cu" "B.Cu") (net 17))
 (segment (start 95.0192 81.38) (end 95.853 81.38) (width 0.127) (layer "B.Cu") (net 17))
 (segment (start 102.2117 74.5474) (end 101.4063 75.3528) (width 0.127) (layer "B.Cu") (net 17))
 (segment (start 102.3935 74.5474) (end 102.2117 74.5474) (width 0.127) (layer "B.Cu") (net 17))
 (segment (start 101.4063 75.3528) (end 101.4063 75.8267) (width 0.127) (layer "B.Cu") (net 17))
 (segment (start 101.4063 75.8267) (end 95.853 81.38) (width 0.127) (layer "B.Cu") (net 17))
 (segment (start 101.9901 75.5945) (end 101.7951 75.3995) (width 0.127) (layer "F.Cu") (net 18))
 (segment (start 101.7951 75.3995) (end 101.7951 68.4379) (width 0.127) (layer "F.Cu") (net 18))
 (segment (start 102.7692 66.63) (end 102.7692 67.4638) (width 0.127) (layer "F.Cu") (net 18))
 (segment (start 101.7951 68.4379) (end 102.7692 67.4638) (width 0.127) (layer "F.Cu") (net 18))
 (via (at 101.9901 75.5945) (size 0.8) (drill 0.4) (layers "F.Cu" "B.Cu") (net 18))
 (segment (start 101.9901 75.5945) (end 95.853 81.7316) (width 0.127) (layer "B.Cu") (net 18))
 (segment (start 95.0192 82.18) (end 95.853 82.18) (width 0.127) (layer "B.Cu") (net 18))
 (segment (start 95.853 81.7316) (end 95.853 82.18) (width 0.127) (layer "B.Cu") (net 18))
 (segment (start 101.0898 68.3432) (end 101.0898 77.4052) (width 0.127) (layer "F.Cu") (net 19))
 (segment (start 101.9692 67.4638) (end 101.0898 68.3432) (width 0.127) (layer "F.Cu") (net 19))
 (segment (start 101.9692 66.63) (end 101.9692 67.4638) (width 0.127) (layer "F.Cu") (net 19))
 (via (at 101.0898 77.4052) (size 0.8) (drill 0.4) (layers "F.Cu" "B.Cu") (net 19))
 (segment (start 95.853 82.642) (end 95.853 82.98) (width 0.127) (layer "B.Cu") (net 19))
 (segment (start 101.0898 77.4052) (end 95.853 82.642) (width 0.127) (layer "B.Cu") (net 19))
 (segment (start 95.0192 82.98) (end 95.853 82.98) (width 0.127) (layer "B.Cu") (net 19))
 (segment (start 100.506 68.127) (end 100.506 78.3255) (width 0.127) (layer "F.Cu") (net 20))
 (segment (start 101.1692 66.63) (end 101.1692 67.4638) (width 0.127) (layer "F.Cu") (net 20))
 (segment (start 100.506 78.3255) (end 100.8431 78.6626) (width 0.127) (layer "F.Cu") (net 20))
 (segment (start 101.1692 67.4638) (end 100.506 68.127) (width 0.127) (layer "F.Cu") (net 20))
 (via (at 100.8431 78.6626) (size 0.8) (drill 0.4) (layers "F.Cu" "B.Cu") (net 20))
 (segment (start 100.6194 78.6626) (end 100.8431 78.6626) (width 0.127) (layer "B.Cu") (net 20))
 (segment (start 95.0192 83.78) (end 95.853 83.78) (width 0.127) (layer "B.Cu") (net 20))
 (segment (start 95.853 83.429) (end 100.6194 78.6626) (width 0.127) (layer "B.Cu") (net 20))
 (segment (start 95.853 83.78) (end 95.853 83.429) (width 0.127) (layer "B.Cu") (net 20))
 (segment (start 100.3692 66.63) (end 100.3692 67.4638) (width 0.127) (layer "F.Cu") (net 21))
 (segment (start 100.3692 67.4638) (end 100.2587 67.5743) (width 0.127) (layer "F.Cu") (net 21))
 (segment (start 100.2587 67.5743) (end 100.2587 79.888) (width 0.127) (layer "F.Cu") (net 21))
 (via (at 100.2587 79.888) (size 0.8) (drill 0.4) (layers "F.Cu" "B.Cu") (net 21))
 (segment (start 96.2844 83.3473) (end 99.7437 79.888) (width 0.127) (layer "B.Cu") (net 21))
 (segment (start 96.2844 84.1486) (end 96.2844 83.3473) (width 0.127) (layer "B.Cu") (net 21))
 (segment (start 95.853 84.58) (end 96.2844 84.1486) (width 0.127) (layer "B.Cu") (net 21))
 (segment (start 99.7437 79.888) (end 100.2587 79.888) (width 0.127) (layer "B.Cu") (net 21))
 (segment (start 95.0192 84.58) (end 95.853 84.58) (width 0.127) (layer "B.Cu") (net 21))
 (segment (start 97.3464 82.0904) (end 97.3464 73.4058) (width 0.127) (layer "F.Cu") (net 22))
 (segment (start 95.0192 85.38) (end 95.853 85.38) (width 0.127) (layer "F.Cu") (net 22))
 (segment (start 97.3464 73.4058) (end 96.919 72.9784) (width 0.127) (layer "F.Cu") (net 22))
 (segment (start 95.853 85.38) (end 95.853 83.5838) (width 0.127) (layer "F.Cu") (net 22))
 (segment (start 95.853 83.5838) (end 97.3464 82.0904) (width 0.127) (layer "F.Cu") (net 22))
 (via (at 96.919 72.9784) (size 0.8) (drill 0.4) (layers "F.Cu" "B.Cu") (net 22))
 (segment (start 99.5692 70.5892) (end 97.18 72.9784) (width 0.127) (layer "B.Cu") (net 22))
 (segment (start 97.18 72.9784) (end 96.919 72.9784) (width 0.127) (layer "B.Cu") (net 22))
 (segment (start 99.5692 66.63) (end 99.5692 70.5892) (width 0.127) (layer "B.Cu") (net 22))
 (segment (start 95.0192 86.18) (end 95.853 86.18) (width 0.127) (layer "F.Cu") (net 23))
 (segment (start 98.1008 72.1419) (end 98.1008 84.0614) (width 0.127) (layer "F.Cu") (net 23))
 (segment (start 95.9822 86.18) (end 95.853 86.18) (width 0.127) (layer "F.Cu") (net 23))
 (segment (start 98.1008 84.0614) (end 95.9822 86.18) (width 0.127) (layer "F.Cu") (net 23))
 (segment (start 97.6426 71.6837) (end 98.1008 72.1419) (width 0.127) (layer "F.Cu") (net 23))
 (via (at 97.6426 71.6837) (size 0.8) (drill 0.4) (layers "F.Cu" "B.Cu") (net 23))
 (segment (start 98.7692 66.63) (end 98.7692 67.4638) (width 0.127) (layer "B.Cu") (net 23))
 (segment (start 98.7692 67.4638) (end 98.9168 67.6114) (width 0.127) (layer "B.Cu") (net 23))
 (segment (start 98.9168 67.6114) (end 98.9168 70.4095) (width 0.127) (layer "B.Cu") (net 23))
 (segment (start 98.9168 70.4095) (end 97.6426 71.6837) (width 0.127) (layer "B.Cu") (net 23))
 (segment (start 97.1197 69.751) (end 97.1197 68.1041) (width 0.127) (layer "F.Cu") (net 24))
 (segment (start 98.6407 71.272) (end 97.1197 69.751) (width 0.127) (layer "F.Cu") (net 24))
 (segment (start 98.6407 85.9538) (end 98.6407 71.272) (width 0.127) (layer "F.Cu") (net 24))
 (segment (start 95.853 86.98) (end 97.6145 86.98) (width 0.127) (layer "F.Cu") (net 24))
 (segment (start 95.0192 86.98) (end 95.853 86.98) (width 0.127) (layer "F.Cu") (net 24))
 (segment (start 97.6145 86.98) (end 98.6407 85.9538) (width 0.127) (layer "F.Cu") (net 24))
 (via (at 97.1197 68.1041) (size 0.8) (drill 0.4) (layers "F.Cu" "B.Cu") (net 24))
 (segment (start 97.76 67.4638) (end 97.1197 68.1041) (width 0.127) (layer "B.Cu") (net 24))
 (segment (start 97.9692 67.4638) (end 97.76 67.4638) (width 0.127) (layer "B.Cu") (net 24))
 (segment (start 97.9692 66.63) (end 97.9692 67.4638) (width 0.127) (layer "B.Cu") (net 24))
 (segment (start 97.1692 88.93) (end 97.1692 88.0962) (width 0.127) (layer "F.Cu") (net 25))
 (segment (start 97.1692 88.0962) (end 98.8995 86.3659) (width 0.127) (layer "F.Cu") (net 25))
 (segment (start 97.1692 66.63) (end 97.1692 67.4638) (width 0.127) (layer "F.Cu") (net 25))
 (segment (start 97.7474 67.8421) (end 97.3691 67.4638) (width 0.127) (layer "F.Cu") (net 25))
 (segment (start 97.3691 67.4638) (end 97.1692 67.4638) (width 0.127) (layer "F.Cu") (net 25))
 (segment (start 98.8995 86.3659) (end 98.8995 71.1811) (width 0.127) (layer "F.Cu") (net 25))
 (segment (start 97.7474 70.029) (end 97.7474 67.8421) (width 0.127) (layer "F.Cu") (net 25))
 (segment (start 98.8995 71.1811) (end 97.7474 70.029) (width 0.127) (layer "F.Cu") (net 25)))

